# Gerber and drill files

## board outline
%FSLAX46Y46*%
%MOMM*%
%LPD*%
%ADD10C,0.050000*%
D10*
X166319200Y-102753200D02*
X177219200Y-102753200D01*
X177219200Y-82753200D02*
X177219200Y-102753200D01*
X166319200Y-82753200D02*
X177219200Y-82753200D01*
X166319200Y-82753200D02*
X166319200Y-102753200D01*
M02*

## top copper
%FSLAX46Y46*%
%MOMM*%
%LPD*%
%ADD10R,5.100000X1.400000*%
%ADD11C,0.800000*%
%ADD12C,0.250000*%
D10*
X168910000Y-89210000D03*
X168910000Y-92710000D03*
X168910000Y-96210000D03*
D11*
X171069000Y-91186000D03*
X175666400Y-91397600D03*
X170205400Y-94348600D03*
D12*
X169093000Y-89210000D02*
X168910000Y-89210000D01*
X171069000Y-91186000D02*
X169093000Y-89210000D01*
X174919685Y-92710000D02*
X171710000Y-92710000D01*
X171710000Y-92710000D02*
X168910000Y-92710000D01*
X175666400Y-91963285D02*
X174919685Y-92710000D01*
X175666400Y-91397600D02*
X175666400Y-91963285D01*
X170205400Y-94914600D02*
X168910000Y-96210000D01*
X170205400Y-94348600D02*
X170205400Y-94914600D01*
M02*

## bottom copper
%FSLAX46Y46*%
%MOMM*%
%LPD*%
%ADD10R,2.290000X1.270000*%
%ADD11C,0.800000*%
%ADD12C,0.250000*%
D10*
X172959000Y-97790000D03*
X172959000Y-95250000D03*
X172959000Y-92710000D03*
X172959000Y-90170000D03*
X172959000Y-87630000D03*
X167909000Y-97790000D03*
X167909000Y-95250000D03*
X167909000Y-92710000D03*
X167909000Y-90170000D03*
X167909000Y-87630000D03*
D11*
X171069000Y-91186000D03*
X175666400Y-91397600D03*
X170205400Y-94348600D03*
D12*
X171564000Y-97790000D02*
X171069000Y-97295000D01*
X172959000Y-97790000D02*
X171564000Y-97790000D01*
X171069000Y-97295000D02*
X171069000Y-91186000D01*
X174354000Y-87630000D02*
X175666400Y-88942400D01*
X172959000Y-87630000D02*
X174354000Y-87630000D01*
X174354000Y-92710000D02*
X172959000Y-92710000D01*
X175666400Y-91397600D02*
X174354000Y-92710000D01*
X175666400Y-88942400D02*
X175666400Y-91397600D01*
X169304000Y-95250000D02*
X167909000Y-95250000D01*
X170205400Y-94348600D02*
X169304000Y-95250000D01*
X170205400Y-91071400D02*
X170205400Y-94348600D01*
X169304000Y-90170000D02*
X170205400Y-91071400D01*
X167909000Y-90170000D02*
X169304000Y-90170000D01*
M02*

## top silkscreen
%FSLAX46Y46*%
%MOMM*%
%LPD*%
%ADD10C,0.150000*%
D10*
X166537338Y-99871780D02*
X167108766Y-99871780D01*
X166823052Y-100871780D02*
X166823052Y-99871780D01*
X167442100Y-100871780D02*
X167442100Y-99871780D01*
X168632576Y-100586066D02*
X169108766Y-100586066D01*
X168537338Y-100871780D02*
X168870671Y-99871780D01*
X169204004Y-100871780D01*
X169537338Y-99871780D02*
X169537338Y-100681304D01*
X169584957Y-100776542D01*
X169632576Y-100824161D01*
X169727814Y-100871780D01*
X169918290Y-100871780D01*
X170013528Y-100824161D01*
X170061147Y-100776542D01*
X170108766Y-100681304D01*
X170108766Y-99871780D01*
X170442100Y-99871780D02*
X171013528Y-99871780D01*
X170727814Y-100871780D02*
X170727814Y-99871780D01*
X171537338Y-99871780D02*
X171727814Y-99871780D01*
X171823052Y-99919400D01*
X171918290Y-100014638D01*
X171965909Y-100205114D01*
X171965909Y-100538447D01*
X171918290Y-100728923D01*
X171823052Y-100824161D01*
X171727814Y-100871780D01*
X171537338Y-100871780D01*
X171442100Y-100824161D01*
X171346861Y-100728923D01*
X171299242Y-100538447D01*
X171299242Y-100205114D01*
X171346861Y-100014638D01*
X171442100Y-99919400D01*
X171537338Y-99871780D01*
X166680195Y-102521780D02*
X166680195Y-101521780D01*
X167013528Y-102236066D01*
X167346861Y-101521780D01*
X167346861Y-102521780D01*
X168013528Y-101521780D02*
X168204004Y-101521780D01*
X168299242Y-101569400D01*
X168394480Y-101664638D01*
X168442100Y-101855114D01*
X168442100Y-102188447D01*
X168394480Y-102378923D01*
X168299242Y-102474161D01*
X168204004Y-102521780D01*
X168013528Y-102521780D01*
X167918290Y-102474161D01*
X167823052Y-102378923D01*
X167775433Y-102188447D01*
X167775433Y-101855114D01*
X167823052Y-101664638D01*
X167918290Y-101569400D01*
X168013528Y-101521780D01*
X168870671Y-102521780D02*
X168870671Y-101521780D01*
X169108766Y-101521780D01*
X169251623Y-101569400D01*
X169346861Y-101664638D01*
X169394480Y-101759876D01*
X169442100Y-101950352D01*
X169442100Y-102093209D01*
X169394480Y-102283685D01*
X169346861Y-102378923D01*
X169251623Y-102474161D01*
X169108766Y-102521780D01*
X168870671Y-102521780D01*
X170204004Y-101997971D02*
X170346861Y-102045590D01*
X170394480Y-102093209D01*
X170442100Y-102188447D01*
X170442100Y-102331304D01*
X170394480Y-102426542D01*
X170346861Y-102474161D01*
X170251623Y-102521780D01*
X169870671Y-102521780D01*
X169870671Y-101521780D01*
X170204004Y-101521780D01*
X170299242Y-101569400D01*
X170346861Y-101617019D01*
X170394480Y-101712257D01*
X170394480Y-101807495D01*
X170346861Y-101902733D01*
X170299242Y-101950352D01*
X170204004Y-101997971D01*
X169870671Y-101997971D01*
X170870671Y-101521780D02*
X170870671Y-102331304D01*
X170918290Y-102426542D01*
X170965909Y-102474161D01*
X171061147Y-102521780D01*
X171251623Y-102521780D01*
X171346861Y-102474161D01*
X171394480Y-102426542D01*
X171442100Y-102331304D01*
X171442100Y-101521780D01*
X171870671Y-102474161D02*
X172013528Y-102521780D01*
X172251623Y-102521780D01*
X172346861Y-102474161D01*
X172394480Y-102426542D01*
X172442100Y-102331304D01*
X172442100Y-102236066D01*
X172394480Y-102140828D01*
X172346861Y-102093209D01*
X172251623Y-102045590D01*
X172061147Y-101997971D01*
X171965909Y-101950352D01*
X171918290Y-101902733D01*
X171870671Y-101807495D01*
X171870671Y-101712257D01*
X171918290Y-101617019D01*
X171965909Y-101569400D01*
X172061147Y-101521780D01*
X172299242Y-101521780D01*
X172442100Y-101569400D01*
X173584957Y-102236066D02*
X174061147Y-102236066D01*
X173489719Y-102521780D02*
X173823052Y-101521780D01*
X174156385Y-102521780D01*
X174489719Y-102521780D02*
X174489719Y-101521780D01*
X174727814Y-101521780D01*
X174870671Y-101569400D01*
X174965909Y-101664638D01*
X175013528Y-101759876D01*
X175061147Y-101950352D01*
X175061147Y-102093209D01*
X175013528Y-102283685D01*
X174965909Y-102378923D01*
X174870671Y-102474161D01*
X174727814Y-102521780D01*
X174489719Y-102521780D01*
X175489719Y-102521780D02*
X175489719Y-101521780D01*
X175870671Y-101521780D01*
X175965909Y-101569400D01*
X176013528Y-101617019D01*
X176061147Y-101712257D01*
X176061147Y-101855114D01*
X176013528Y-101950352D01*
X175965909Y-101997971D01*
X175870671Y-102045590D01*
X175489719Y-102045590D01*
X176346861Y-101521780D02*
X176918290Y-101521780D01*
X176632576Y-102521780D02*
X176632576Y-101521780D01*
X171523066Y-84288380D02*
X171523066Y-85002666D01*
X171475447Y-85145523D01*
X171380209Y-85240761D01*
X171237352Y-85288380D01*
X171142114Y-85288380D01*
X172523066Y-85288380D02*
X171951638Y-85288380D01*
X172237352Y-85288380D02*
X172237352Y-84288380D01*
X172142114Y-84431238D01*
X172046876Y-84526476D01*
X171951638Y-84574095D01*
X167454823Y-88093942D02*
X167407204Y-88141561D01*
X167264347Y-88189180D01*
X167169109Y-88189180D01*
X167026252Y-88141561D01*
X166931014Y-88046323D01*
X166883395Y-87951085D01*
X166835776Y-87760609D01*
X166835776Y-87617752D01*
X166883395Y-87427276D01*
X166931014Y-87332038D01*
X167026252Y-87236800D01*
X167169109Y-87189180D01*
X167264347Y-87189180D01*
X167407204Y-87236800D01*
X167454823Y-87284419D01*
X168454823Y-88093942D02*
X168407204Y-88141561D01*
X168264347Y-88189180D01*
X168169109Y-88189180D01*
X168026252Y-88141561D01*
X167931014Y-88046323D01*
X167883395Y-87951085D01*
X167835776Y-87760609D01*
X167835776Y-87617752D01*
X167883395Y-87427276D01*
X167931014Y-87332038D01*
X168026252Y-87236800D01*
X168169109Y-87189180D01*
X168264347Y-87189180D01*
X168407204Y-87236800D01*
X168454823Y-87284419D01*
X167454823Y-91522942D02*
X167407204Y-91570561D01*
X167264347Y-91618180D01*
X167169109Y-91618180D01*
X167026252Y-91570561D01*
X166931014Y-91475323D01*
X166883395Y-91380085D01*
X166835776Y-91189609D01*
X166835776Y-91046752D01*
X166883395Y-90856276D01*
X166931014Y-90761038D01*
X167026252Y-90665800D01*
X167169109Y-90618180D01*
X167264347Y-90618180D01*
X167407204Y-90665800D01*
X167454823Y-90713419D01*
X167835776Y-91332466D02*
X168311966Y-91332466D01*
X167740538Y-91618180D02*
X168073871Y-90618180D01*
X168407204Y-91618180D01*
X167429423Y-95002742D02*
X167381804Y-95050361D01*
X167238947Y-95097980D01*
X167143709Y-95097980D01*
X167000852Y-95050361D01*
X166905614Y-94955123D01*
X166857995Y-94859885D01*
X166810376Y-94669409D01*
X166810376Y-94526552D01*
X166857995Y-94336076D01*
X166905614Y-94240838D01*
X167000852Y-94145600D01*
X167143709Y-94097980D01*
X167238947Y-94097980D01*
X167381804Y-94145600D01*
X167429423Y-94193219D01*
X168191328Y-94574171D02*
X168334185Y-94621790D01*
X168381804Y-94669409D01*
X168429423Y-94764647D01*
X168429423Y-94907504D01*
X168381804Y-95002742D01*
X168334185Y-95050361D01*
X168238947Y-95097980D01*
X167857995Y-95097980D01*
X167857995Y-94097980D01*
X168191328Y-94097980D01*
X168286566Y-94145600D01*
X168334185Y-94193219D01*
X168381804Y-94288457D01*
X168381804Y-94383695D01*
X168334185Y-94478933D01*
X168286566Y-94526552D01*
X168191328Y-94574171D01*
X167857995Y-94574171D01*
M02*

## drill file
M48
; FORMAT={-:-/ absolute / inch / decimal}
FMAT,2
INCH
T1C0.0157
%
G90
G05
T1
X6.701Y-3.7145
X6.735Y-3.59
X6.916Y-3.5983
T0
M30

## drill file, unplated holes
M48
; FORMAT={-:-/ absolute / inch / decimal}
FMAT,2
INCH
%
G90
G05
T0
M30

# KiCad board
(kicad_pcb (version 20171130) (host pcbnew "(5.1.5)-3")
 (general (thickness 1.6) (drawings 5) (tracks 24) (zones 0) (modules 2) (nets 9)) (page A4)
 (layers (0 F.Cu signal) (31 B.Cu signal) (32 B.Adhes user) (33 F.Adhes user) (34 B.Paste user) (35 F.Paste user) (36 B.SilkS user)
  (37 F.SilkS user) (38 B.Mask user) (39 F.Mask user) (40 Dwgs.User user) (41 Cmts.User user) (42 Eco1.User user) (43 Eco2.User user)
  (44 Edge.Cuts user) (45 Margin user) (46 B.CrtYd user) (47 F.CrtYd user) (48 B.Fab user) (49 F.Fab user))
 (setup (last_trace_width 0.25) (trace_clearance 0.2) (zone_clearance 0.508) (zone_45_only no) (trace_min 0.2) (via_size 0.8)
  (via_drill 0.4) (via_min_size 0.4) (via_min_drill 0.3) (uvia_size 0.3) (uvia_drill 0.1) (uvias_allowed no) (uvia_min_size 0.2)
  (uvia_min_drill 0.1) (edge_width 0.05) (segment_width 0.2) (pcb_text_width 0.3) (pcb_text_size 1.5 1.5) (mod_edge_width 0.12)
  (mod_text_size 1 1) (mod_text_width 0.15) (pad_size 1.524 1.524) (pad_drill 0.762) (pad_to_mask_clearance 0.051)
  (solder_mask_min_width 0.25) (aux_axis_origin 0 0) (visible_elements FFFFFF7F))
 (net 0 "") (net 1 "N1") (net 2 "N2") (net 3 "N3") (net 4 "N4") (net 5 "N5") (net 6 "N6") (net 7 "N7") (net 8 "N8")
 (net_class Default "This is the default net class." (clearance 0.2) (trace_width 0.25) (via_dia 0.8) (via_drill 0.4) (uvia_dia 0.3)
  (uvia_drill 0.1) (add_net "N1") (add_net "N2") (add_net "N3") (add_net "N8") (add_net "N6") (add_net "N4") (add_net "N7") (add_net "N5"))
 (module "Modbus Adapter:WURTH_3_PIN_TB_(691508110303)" (layer F.Cu) (at 166.3192 85.8318)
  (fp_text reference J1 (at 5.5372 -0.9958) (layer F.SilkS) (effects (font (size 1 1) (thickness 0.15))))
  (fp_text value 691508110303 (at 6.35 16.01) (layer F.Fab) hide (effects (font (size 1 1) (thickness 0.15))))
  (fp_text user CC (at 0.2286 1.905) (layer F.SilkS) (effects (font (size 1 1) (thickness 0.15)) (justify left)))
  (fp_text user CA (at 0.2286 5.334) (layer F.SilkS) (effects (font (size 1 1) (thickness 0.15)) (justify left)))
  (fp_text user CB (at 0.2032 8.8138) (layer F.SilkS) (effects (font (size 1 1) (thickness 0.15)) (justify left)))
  (pad 1 smd rect (at 2.5908 3.3782 270) (size 1.4 5.1) (layers F.Cu F.Paste F.Mask) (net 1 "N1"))
  (pad 2 smd rect (at 2.5908 6.8782 270) (size 1.4 5.1) (layers F.Cu F.Paste F.Mask) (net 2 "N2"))
  (pad 3 smd rect (at 2.5908 10.3782 270) (size 1.4 5.1) (layers F.Cu F.Paste F.Mask) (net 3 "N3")))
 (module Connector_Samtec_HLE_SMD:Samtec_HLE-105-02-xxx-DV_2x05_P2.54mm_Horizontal (layer B.Cu) (at 170.434 92.71 90)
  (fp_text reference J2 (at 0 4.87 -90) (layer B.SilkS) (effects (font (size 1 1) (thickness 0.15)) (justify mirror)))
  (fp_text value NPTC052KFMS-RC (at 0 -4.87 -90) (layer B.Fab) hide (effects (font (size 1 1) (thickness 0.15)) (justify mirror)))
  (pad 1 smd rect (at -5.08 2.525 90) (size 1.27 2.29) (layers B.Cu B.Paste B.Mask) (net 1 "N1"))
  (pad 3 smd rect (at -2.54 2.525 90) (size 1.27 2.29) (layers B.Cu B.Paste B.Mask) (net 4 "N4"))
  (pad 5 smd rect (at 0 2.525 90) (size 1.27 2.29) (layers B.Cu B.Paste B.Mask) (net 2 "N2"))
  (pad 7 smd rect (at 2.54 2.525 90) (size 1.27 2.29) (layers B.Cu B.Paste B.Mask) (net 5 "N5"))
  (pad 9 smd rect (at 5.08 2.525 90) (size 1.27 2.29) (layers B.Cu B.Paste B.Mask) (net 2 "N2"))
  (pad 2 smd rect (at -5.08 -2.525 90) (size 1.27 2.29) (layers B.Cu B.Paste B.Mask) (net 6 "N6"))
  (pad 4 smd rect (at -2.54 -2.525 90) (size 1.27 2.29) (layers B.Cu B.Paste B.Mask) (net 3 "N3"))
  (pad 6 smd rect (at 0 -2.525 90) (size 1.27 2.29) (layers B.Cu B.Paste B.Mask) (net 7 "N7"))
  (pad 8 smd rect (at 2.54 -2.525 90) (size 1.27 2.29) (layers B.Cu B.Paste B.Mask) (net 3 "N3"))
  (pad 10 smd rect (at 5.08 -2.525 90) (size 1.27 2.29) (layers B.Cu B.Paste B.Mask) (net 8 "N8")))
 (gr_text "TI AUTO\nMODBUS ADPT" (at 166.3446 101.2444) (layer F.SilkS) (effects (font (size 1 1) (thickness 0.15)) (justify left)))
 (gr_line (start 166.3192 102.7532) (end 177.2192 102.7532) (layer Edge.Cuts) (width 0.05))
 (gr_line (start 177.2192 82.7532) (end 177.2192 102.7532) (layer Edge.Cuts) (width 0.05))
 (gr_line (start 166.3192 82.7532) (end 177.2192 82.7532) (layer Edge.Cuts) (width 0.05))
 (gr_line (start 166.3192 82.7532) (end 166.3192 102.7532) (layer Edge.Cuts) (width 0.05))
 (segment (start 171.564 97.79) (end 171.069 97.295) (width 0.25) (layer B.Cu) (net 1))
 (segment (start 172.959 97.79) (end 171.564 97.79) (width 0.25) (layer B.Cu) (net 1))
 (via (at 171.069 91.186) (size 0.8) (drill 0.4) (layers F.Cu B.Cu) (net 1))
 (segment (start 171.069 97.295) (end 171.069 91.186) (width 0.25) (layer B.Cu) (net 1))
 (segment (start 169.093 89.21) (end 168.91 89.21) (width 0.25) (layer F.Cu) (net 1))
 (segment (start 171.069 91.186) (end 169.093 89.21) (width 0.25) (layer F.Cu) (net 1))
 (segment (start 174.354 87.63) (end 175.6664 88.9424) (width 0.25) (layer B.Cu) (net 2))
 (segment (start 172.959 87.63) (end 174.354 87.63) (width 0.25) (layer B.Cu) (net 2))
 (segment (start 174.354 92.71) (end 172.959 92.71) (width 0.25) (layer B.Cu) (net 2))
 (segment (start 175.6664 91.3976) (end 174.354 92.71) (width 0.25) (layer B.Cu) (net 2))
 (segment (start 175.6664 88.9424) (end 175.6664 91.3976) (width 0.25) (layer B.Cu) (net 2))
 (via (at 175.6664 91.3976) (size 0.8) (drill 0.4) (layers F.Cu B.Cu) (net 2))
 (segment (start 174.919685 92.71) (end 171.71 92.71) (width 0.25) (layer F.Cu) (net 2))
 (segment (start 171.71 92.71) (end 168.91 92.71) (width 0.25) (layer F.Cu) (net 2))
 (segment (start 175.6664 91.963285) (end 174.919685 92.71) (width 0.25) (layer F.Cu) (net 2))
 (segment (start 175.6664 91.3976) (end 175.6664 91.963285) (width 0.25) (layer F.Cu) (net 2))
 (segment (start 169.304 95.25) (end 167.909 95.25) (width 0.25) (layer B.Cu) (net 3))
 (segment (start 170.2054 94.3486) (end 169.304 95.25) (width 0.25) (layer B.Cu) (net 3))
 (segment (start 170.2054 91.0714) (end 170.2054 94.3486) (width 0.25) (layer B.Cu) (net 3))
 (segment (start 169.304 90.17) (end 170.2054 91.0714) (width 0.25) (layer B.Cu) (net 3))
 (segment (start 167.909 90.17) (end 169.304 90.17) (width 0.25) (layer B.Cu) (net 3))
 (via (at 170.2054 94.3486) (size 0.8) (drill 0.4) (layers F.Cu B.Cu) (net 3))
 (segment (start 170.2054 94.9146) (end 168.91 96.21) (width 0.25) (layer F.Cu) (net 3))
 (segment (start 170.2054 94.3486) (end 170.2054 94.9146) (width 0.25) (layer F.Cu) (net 3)))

